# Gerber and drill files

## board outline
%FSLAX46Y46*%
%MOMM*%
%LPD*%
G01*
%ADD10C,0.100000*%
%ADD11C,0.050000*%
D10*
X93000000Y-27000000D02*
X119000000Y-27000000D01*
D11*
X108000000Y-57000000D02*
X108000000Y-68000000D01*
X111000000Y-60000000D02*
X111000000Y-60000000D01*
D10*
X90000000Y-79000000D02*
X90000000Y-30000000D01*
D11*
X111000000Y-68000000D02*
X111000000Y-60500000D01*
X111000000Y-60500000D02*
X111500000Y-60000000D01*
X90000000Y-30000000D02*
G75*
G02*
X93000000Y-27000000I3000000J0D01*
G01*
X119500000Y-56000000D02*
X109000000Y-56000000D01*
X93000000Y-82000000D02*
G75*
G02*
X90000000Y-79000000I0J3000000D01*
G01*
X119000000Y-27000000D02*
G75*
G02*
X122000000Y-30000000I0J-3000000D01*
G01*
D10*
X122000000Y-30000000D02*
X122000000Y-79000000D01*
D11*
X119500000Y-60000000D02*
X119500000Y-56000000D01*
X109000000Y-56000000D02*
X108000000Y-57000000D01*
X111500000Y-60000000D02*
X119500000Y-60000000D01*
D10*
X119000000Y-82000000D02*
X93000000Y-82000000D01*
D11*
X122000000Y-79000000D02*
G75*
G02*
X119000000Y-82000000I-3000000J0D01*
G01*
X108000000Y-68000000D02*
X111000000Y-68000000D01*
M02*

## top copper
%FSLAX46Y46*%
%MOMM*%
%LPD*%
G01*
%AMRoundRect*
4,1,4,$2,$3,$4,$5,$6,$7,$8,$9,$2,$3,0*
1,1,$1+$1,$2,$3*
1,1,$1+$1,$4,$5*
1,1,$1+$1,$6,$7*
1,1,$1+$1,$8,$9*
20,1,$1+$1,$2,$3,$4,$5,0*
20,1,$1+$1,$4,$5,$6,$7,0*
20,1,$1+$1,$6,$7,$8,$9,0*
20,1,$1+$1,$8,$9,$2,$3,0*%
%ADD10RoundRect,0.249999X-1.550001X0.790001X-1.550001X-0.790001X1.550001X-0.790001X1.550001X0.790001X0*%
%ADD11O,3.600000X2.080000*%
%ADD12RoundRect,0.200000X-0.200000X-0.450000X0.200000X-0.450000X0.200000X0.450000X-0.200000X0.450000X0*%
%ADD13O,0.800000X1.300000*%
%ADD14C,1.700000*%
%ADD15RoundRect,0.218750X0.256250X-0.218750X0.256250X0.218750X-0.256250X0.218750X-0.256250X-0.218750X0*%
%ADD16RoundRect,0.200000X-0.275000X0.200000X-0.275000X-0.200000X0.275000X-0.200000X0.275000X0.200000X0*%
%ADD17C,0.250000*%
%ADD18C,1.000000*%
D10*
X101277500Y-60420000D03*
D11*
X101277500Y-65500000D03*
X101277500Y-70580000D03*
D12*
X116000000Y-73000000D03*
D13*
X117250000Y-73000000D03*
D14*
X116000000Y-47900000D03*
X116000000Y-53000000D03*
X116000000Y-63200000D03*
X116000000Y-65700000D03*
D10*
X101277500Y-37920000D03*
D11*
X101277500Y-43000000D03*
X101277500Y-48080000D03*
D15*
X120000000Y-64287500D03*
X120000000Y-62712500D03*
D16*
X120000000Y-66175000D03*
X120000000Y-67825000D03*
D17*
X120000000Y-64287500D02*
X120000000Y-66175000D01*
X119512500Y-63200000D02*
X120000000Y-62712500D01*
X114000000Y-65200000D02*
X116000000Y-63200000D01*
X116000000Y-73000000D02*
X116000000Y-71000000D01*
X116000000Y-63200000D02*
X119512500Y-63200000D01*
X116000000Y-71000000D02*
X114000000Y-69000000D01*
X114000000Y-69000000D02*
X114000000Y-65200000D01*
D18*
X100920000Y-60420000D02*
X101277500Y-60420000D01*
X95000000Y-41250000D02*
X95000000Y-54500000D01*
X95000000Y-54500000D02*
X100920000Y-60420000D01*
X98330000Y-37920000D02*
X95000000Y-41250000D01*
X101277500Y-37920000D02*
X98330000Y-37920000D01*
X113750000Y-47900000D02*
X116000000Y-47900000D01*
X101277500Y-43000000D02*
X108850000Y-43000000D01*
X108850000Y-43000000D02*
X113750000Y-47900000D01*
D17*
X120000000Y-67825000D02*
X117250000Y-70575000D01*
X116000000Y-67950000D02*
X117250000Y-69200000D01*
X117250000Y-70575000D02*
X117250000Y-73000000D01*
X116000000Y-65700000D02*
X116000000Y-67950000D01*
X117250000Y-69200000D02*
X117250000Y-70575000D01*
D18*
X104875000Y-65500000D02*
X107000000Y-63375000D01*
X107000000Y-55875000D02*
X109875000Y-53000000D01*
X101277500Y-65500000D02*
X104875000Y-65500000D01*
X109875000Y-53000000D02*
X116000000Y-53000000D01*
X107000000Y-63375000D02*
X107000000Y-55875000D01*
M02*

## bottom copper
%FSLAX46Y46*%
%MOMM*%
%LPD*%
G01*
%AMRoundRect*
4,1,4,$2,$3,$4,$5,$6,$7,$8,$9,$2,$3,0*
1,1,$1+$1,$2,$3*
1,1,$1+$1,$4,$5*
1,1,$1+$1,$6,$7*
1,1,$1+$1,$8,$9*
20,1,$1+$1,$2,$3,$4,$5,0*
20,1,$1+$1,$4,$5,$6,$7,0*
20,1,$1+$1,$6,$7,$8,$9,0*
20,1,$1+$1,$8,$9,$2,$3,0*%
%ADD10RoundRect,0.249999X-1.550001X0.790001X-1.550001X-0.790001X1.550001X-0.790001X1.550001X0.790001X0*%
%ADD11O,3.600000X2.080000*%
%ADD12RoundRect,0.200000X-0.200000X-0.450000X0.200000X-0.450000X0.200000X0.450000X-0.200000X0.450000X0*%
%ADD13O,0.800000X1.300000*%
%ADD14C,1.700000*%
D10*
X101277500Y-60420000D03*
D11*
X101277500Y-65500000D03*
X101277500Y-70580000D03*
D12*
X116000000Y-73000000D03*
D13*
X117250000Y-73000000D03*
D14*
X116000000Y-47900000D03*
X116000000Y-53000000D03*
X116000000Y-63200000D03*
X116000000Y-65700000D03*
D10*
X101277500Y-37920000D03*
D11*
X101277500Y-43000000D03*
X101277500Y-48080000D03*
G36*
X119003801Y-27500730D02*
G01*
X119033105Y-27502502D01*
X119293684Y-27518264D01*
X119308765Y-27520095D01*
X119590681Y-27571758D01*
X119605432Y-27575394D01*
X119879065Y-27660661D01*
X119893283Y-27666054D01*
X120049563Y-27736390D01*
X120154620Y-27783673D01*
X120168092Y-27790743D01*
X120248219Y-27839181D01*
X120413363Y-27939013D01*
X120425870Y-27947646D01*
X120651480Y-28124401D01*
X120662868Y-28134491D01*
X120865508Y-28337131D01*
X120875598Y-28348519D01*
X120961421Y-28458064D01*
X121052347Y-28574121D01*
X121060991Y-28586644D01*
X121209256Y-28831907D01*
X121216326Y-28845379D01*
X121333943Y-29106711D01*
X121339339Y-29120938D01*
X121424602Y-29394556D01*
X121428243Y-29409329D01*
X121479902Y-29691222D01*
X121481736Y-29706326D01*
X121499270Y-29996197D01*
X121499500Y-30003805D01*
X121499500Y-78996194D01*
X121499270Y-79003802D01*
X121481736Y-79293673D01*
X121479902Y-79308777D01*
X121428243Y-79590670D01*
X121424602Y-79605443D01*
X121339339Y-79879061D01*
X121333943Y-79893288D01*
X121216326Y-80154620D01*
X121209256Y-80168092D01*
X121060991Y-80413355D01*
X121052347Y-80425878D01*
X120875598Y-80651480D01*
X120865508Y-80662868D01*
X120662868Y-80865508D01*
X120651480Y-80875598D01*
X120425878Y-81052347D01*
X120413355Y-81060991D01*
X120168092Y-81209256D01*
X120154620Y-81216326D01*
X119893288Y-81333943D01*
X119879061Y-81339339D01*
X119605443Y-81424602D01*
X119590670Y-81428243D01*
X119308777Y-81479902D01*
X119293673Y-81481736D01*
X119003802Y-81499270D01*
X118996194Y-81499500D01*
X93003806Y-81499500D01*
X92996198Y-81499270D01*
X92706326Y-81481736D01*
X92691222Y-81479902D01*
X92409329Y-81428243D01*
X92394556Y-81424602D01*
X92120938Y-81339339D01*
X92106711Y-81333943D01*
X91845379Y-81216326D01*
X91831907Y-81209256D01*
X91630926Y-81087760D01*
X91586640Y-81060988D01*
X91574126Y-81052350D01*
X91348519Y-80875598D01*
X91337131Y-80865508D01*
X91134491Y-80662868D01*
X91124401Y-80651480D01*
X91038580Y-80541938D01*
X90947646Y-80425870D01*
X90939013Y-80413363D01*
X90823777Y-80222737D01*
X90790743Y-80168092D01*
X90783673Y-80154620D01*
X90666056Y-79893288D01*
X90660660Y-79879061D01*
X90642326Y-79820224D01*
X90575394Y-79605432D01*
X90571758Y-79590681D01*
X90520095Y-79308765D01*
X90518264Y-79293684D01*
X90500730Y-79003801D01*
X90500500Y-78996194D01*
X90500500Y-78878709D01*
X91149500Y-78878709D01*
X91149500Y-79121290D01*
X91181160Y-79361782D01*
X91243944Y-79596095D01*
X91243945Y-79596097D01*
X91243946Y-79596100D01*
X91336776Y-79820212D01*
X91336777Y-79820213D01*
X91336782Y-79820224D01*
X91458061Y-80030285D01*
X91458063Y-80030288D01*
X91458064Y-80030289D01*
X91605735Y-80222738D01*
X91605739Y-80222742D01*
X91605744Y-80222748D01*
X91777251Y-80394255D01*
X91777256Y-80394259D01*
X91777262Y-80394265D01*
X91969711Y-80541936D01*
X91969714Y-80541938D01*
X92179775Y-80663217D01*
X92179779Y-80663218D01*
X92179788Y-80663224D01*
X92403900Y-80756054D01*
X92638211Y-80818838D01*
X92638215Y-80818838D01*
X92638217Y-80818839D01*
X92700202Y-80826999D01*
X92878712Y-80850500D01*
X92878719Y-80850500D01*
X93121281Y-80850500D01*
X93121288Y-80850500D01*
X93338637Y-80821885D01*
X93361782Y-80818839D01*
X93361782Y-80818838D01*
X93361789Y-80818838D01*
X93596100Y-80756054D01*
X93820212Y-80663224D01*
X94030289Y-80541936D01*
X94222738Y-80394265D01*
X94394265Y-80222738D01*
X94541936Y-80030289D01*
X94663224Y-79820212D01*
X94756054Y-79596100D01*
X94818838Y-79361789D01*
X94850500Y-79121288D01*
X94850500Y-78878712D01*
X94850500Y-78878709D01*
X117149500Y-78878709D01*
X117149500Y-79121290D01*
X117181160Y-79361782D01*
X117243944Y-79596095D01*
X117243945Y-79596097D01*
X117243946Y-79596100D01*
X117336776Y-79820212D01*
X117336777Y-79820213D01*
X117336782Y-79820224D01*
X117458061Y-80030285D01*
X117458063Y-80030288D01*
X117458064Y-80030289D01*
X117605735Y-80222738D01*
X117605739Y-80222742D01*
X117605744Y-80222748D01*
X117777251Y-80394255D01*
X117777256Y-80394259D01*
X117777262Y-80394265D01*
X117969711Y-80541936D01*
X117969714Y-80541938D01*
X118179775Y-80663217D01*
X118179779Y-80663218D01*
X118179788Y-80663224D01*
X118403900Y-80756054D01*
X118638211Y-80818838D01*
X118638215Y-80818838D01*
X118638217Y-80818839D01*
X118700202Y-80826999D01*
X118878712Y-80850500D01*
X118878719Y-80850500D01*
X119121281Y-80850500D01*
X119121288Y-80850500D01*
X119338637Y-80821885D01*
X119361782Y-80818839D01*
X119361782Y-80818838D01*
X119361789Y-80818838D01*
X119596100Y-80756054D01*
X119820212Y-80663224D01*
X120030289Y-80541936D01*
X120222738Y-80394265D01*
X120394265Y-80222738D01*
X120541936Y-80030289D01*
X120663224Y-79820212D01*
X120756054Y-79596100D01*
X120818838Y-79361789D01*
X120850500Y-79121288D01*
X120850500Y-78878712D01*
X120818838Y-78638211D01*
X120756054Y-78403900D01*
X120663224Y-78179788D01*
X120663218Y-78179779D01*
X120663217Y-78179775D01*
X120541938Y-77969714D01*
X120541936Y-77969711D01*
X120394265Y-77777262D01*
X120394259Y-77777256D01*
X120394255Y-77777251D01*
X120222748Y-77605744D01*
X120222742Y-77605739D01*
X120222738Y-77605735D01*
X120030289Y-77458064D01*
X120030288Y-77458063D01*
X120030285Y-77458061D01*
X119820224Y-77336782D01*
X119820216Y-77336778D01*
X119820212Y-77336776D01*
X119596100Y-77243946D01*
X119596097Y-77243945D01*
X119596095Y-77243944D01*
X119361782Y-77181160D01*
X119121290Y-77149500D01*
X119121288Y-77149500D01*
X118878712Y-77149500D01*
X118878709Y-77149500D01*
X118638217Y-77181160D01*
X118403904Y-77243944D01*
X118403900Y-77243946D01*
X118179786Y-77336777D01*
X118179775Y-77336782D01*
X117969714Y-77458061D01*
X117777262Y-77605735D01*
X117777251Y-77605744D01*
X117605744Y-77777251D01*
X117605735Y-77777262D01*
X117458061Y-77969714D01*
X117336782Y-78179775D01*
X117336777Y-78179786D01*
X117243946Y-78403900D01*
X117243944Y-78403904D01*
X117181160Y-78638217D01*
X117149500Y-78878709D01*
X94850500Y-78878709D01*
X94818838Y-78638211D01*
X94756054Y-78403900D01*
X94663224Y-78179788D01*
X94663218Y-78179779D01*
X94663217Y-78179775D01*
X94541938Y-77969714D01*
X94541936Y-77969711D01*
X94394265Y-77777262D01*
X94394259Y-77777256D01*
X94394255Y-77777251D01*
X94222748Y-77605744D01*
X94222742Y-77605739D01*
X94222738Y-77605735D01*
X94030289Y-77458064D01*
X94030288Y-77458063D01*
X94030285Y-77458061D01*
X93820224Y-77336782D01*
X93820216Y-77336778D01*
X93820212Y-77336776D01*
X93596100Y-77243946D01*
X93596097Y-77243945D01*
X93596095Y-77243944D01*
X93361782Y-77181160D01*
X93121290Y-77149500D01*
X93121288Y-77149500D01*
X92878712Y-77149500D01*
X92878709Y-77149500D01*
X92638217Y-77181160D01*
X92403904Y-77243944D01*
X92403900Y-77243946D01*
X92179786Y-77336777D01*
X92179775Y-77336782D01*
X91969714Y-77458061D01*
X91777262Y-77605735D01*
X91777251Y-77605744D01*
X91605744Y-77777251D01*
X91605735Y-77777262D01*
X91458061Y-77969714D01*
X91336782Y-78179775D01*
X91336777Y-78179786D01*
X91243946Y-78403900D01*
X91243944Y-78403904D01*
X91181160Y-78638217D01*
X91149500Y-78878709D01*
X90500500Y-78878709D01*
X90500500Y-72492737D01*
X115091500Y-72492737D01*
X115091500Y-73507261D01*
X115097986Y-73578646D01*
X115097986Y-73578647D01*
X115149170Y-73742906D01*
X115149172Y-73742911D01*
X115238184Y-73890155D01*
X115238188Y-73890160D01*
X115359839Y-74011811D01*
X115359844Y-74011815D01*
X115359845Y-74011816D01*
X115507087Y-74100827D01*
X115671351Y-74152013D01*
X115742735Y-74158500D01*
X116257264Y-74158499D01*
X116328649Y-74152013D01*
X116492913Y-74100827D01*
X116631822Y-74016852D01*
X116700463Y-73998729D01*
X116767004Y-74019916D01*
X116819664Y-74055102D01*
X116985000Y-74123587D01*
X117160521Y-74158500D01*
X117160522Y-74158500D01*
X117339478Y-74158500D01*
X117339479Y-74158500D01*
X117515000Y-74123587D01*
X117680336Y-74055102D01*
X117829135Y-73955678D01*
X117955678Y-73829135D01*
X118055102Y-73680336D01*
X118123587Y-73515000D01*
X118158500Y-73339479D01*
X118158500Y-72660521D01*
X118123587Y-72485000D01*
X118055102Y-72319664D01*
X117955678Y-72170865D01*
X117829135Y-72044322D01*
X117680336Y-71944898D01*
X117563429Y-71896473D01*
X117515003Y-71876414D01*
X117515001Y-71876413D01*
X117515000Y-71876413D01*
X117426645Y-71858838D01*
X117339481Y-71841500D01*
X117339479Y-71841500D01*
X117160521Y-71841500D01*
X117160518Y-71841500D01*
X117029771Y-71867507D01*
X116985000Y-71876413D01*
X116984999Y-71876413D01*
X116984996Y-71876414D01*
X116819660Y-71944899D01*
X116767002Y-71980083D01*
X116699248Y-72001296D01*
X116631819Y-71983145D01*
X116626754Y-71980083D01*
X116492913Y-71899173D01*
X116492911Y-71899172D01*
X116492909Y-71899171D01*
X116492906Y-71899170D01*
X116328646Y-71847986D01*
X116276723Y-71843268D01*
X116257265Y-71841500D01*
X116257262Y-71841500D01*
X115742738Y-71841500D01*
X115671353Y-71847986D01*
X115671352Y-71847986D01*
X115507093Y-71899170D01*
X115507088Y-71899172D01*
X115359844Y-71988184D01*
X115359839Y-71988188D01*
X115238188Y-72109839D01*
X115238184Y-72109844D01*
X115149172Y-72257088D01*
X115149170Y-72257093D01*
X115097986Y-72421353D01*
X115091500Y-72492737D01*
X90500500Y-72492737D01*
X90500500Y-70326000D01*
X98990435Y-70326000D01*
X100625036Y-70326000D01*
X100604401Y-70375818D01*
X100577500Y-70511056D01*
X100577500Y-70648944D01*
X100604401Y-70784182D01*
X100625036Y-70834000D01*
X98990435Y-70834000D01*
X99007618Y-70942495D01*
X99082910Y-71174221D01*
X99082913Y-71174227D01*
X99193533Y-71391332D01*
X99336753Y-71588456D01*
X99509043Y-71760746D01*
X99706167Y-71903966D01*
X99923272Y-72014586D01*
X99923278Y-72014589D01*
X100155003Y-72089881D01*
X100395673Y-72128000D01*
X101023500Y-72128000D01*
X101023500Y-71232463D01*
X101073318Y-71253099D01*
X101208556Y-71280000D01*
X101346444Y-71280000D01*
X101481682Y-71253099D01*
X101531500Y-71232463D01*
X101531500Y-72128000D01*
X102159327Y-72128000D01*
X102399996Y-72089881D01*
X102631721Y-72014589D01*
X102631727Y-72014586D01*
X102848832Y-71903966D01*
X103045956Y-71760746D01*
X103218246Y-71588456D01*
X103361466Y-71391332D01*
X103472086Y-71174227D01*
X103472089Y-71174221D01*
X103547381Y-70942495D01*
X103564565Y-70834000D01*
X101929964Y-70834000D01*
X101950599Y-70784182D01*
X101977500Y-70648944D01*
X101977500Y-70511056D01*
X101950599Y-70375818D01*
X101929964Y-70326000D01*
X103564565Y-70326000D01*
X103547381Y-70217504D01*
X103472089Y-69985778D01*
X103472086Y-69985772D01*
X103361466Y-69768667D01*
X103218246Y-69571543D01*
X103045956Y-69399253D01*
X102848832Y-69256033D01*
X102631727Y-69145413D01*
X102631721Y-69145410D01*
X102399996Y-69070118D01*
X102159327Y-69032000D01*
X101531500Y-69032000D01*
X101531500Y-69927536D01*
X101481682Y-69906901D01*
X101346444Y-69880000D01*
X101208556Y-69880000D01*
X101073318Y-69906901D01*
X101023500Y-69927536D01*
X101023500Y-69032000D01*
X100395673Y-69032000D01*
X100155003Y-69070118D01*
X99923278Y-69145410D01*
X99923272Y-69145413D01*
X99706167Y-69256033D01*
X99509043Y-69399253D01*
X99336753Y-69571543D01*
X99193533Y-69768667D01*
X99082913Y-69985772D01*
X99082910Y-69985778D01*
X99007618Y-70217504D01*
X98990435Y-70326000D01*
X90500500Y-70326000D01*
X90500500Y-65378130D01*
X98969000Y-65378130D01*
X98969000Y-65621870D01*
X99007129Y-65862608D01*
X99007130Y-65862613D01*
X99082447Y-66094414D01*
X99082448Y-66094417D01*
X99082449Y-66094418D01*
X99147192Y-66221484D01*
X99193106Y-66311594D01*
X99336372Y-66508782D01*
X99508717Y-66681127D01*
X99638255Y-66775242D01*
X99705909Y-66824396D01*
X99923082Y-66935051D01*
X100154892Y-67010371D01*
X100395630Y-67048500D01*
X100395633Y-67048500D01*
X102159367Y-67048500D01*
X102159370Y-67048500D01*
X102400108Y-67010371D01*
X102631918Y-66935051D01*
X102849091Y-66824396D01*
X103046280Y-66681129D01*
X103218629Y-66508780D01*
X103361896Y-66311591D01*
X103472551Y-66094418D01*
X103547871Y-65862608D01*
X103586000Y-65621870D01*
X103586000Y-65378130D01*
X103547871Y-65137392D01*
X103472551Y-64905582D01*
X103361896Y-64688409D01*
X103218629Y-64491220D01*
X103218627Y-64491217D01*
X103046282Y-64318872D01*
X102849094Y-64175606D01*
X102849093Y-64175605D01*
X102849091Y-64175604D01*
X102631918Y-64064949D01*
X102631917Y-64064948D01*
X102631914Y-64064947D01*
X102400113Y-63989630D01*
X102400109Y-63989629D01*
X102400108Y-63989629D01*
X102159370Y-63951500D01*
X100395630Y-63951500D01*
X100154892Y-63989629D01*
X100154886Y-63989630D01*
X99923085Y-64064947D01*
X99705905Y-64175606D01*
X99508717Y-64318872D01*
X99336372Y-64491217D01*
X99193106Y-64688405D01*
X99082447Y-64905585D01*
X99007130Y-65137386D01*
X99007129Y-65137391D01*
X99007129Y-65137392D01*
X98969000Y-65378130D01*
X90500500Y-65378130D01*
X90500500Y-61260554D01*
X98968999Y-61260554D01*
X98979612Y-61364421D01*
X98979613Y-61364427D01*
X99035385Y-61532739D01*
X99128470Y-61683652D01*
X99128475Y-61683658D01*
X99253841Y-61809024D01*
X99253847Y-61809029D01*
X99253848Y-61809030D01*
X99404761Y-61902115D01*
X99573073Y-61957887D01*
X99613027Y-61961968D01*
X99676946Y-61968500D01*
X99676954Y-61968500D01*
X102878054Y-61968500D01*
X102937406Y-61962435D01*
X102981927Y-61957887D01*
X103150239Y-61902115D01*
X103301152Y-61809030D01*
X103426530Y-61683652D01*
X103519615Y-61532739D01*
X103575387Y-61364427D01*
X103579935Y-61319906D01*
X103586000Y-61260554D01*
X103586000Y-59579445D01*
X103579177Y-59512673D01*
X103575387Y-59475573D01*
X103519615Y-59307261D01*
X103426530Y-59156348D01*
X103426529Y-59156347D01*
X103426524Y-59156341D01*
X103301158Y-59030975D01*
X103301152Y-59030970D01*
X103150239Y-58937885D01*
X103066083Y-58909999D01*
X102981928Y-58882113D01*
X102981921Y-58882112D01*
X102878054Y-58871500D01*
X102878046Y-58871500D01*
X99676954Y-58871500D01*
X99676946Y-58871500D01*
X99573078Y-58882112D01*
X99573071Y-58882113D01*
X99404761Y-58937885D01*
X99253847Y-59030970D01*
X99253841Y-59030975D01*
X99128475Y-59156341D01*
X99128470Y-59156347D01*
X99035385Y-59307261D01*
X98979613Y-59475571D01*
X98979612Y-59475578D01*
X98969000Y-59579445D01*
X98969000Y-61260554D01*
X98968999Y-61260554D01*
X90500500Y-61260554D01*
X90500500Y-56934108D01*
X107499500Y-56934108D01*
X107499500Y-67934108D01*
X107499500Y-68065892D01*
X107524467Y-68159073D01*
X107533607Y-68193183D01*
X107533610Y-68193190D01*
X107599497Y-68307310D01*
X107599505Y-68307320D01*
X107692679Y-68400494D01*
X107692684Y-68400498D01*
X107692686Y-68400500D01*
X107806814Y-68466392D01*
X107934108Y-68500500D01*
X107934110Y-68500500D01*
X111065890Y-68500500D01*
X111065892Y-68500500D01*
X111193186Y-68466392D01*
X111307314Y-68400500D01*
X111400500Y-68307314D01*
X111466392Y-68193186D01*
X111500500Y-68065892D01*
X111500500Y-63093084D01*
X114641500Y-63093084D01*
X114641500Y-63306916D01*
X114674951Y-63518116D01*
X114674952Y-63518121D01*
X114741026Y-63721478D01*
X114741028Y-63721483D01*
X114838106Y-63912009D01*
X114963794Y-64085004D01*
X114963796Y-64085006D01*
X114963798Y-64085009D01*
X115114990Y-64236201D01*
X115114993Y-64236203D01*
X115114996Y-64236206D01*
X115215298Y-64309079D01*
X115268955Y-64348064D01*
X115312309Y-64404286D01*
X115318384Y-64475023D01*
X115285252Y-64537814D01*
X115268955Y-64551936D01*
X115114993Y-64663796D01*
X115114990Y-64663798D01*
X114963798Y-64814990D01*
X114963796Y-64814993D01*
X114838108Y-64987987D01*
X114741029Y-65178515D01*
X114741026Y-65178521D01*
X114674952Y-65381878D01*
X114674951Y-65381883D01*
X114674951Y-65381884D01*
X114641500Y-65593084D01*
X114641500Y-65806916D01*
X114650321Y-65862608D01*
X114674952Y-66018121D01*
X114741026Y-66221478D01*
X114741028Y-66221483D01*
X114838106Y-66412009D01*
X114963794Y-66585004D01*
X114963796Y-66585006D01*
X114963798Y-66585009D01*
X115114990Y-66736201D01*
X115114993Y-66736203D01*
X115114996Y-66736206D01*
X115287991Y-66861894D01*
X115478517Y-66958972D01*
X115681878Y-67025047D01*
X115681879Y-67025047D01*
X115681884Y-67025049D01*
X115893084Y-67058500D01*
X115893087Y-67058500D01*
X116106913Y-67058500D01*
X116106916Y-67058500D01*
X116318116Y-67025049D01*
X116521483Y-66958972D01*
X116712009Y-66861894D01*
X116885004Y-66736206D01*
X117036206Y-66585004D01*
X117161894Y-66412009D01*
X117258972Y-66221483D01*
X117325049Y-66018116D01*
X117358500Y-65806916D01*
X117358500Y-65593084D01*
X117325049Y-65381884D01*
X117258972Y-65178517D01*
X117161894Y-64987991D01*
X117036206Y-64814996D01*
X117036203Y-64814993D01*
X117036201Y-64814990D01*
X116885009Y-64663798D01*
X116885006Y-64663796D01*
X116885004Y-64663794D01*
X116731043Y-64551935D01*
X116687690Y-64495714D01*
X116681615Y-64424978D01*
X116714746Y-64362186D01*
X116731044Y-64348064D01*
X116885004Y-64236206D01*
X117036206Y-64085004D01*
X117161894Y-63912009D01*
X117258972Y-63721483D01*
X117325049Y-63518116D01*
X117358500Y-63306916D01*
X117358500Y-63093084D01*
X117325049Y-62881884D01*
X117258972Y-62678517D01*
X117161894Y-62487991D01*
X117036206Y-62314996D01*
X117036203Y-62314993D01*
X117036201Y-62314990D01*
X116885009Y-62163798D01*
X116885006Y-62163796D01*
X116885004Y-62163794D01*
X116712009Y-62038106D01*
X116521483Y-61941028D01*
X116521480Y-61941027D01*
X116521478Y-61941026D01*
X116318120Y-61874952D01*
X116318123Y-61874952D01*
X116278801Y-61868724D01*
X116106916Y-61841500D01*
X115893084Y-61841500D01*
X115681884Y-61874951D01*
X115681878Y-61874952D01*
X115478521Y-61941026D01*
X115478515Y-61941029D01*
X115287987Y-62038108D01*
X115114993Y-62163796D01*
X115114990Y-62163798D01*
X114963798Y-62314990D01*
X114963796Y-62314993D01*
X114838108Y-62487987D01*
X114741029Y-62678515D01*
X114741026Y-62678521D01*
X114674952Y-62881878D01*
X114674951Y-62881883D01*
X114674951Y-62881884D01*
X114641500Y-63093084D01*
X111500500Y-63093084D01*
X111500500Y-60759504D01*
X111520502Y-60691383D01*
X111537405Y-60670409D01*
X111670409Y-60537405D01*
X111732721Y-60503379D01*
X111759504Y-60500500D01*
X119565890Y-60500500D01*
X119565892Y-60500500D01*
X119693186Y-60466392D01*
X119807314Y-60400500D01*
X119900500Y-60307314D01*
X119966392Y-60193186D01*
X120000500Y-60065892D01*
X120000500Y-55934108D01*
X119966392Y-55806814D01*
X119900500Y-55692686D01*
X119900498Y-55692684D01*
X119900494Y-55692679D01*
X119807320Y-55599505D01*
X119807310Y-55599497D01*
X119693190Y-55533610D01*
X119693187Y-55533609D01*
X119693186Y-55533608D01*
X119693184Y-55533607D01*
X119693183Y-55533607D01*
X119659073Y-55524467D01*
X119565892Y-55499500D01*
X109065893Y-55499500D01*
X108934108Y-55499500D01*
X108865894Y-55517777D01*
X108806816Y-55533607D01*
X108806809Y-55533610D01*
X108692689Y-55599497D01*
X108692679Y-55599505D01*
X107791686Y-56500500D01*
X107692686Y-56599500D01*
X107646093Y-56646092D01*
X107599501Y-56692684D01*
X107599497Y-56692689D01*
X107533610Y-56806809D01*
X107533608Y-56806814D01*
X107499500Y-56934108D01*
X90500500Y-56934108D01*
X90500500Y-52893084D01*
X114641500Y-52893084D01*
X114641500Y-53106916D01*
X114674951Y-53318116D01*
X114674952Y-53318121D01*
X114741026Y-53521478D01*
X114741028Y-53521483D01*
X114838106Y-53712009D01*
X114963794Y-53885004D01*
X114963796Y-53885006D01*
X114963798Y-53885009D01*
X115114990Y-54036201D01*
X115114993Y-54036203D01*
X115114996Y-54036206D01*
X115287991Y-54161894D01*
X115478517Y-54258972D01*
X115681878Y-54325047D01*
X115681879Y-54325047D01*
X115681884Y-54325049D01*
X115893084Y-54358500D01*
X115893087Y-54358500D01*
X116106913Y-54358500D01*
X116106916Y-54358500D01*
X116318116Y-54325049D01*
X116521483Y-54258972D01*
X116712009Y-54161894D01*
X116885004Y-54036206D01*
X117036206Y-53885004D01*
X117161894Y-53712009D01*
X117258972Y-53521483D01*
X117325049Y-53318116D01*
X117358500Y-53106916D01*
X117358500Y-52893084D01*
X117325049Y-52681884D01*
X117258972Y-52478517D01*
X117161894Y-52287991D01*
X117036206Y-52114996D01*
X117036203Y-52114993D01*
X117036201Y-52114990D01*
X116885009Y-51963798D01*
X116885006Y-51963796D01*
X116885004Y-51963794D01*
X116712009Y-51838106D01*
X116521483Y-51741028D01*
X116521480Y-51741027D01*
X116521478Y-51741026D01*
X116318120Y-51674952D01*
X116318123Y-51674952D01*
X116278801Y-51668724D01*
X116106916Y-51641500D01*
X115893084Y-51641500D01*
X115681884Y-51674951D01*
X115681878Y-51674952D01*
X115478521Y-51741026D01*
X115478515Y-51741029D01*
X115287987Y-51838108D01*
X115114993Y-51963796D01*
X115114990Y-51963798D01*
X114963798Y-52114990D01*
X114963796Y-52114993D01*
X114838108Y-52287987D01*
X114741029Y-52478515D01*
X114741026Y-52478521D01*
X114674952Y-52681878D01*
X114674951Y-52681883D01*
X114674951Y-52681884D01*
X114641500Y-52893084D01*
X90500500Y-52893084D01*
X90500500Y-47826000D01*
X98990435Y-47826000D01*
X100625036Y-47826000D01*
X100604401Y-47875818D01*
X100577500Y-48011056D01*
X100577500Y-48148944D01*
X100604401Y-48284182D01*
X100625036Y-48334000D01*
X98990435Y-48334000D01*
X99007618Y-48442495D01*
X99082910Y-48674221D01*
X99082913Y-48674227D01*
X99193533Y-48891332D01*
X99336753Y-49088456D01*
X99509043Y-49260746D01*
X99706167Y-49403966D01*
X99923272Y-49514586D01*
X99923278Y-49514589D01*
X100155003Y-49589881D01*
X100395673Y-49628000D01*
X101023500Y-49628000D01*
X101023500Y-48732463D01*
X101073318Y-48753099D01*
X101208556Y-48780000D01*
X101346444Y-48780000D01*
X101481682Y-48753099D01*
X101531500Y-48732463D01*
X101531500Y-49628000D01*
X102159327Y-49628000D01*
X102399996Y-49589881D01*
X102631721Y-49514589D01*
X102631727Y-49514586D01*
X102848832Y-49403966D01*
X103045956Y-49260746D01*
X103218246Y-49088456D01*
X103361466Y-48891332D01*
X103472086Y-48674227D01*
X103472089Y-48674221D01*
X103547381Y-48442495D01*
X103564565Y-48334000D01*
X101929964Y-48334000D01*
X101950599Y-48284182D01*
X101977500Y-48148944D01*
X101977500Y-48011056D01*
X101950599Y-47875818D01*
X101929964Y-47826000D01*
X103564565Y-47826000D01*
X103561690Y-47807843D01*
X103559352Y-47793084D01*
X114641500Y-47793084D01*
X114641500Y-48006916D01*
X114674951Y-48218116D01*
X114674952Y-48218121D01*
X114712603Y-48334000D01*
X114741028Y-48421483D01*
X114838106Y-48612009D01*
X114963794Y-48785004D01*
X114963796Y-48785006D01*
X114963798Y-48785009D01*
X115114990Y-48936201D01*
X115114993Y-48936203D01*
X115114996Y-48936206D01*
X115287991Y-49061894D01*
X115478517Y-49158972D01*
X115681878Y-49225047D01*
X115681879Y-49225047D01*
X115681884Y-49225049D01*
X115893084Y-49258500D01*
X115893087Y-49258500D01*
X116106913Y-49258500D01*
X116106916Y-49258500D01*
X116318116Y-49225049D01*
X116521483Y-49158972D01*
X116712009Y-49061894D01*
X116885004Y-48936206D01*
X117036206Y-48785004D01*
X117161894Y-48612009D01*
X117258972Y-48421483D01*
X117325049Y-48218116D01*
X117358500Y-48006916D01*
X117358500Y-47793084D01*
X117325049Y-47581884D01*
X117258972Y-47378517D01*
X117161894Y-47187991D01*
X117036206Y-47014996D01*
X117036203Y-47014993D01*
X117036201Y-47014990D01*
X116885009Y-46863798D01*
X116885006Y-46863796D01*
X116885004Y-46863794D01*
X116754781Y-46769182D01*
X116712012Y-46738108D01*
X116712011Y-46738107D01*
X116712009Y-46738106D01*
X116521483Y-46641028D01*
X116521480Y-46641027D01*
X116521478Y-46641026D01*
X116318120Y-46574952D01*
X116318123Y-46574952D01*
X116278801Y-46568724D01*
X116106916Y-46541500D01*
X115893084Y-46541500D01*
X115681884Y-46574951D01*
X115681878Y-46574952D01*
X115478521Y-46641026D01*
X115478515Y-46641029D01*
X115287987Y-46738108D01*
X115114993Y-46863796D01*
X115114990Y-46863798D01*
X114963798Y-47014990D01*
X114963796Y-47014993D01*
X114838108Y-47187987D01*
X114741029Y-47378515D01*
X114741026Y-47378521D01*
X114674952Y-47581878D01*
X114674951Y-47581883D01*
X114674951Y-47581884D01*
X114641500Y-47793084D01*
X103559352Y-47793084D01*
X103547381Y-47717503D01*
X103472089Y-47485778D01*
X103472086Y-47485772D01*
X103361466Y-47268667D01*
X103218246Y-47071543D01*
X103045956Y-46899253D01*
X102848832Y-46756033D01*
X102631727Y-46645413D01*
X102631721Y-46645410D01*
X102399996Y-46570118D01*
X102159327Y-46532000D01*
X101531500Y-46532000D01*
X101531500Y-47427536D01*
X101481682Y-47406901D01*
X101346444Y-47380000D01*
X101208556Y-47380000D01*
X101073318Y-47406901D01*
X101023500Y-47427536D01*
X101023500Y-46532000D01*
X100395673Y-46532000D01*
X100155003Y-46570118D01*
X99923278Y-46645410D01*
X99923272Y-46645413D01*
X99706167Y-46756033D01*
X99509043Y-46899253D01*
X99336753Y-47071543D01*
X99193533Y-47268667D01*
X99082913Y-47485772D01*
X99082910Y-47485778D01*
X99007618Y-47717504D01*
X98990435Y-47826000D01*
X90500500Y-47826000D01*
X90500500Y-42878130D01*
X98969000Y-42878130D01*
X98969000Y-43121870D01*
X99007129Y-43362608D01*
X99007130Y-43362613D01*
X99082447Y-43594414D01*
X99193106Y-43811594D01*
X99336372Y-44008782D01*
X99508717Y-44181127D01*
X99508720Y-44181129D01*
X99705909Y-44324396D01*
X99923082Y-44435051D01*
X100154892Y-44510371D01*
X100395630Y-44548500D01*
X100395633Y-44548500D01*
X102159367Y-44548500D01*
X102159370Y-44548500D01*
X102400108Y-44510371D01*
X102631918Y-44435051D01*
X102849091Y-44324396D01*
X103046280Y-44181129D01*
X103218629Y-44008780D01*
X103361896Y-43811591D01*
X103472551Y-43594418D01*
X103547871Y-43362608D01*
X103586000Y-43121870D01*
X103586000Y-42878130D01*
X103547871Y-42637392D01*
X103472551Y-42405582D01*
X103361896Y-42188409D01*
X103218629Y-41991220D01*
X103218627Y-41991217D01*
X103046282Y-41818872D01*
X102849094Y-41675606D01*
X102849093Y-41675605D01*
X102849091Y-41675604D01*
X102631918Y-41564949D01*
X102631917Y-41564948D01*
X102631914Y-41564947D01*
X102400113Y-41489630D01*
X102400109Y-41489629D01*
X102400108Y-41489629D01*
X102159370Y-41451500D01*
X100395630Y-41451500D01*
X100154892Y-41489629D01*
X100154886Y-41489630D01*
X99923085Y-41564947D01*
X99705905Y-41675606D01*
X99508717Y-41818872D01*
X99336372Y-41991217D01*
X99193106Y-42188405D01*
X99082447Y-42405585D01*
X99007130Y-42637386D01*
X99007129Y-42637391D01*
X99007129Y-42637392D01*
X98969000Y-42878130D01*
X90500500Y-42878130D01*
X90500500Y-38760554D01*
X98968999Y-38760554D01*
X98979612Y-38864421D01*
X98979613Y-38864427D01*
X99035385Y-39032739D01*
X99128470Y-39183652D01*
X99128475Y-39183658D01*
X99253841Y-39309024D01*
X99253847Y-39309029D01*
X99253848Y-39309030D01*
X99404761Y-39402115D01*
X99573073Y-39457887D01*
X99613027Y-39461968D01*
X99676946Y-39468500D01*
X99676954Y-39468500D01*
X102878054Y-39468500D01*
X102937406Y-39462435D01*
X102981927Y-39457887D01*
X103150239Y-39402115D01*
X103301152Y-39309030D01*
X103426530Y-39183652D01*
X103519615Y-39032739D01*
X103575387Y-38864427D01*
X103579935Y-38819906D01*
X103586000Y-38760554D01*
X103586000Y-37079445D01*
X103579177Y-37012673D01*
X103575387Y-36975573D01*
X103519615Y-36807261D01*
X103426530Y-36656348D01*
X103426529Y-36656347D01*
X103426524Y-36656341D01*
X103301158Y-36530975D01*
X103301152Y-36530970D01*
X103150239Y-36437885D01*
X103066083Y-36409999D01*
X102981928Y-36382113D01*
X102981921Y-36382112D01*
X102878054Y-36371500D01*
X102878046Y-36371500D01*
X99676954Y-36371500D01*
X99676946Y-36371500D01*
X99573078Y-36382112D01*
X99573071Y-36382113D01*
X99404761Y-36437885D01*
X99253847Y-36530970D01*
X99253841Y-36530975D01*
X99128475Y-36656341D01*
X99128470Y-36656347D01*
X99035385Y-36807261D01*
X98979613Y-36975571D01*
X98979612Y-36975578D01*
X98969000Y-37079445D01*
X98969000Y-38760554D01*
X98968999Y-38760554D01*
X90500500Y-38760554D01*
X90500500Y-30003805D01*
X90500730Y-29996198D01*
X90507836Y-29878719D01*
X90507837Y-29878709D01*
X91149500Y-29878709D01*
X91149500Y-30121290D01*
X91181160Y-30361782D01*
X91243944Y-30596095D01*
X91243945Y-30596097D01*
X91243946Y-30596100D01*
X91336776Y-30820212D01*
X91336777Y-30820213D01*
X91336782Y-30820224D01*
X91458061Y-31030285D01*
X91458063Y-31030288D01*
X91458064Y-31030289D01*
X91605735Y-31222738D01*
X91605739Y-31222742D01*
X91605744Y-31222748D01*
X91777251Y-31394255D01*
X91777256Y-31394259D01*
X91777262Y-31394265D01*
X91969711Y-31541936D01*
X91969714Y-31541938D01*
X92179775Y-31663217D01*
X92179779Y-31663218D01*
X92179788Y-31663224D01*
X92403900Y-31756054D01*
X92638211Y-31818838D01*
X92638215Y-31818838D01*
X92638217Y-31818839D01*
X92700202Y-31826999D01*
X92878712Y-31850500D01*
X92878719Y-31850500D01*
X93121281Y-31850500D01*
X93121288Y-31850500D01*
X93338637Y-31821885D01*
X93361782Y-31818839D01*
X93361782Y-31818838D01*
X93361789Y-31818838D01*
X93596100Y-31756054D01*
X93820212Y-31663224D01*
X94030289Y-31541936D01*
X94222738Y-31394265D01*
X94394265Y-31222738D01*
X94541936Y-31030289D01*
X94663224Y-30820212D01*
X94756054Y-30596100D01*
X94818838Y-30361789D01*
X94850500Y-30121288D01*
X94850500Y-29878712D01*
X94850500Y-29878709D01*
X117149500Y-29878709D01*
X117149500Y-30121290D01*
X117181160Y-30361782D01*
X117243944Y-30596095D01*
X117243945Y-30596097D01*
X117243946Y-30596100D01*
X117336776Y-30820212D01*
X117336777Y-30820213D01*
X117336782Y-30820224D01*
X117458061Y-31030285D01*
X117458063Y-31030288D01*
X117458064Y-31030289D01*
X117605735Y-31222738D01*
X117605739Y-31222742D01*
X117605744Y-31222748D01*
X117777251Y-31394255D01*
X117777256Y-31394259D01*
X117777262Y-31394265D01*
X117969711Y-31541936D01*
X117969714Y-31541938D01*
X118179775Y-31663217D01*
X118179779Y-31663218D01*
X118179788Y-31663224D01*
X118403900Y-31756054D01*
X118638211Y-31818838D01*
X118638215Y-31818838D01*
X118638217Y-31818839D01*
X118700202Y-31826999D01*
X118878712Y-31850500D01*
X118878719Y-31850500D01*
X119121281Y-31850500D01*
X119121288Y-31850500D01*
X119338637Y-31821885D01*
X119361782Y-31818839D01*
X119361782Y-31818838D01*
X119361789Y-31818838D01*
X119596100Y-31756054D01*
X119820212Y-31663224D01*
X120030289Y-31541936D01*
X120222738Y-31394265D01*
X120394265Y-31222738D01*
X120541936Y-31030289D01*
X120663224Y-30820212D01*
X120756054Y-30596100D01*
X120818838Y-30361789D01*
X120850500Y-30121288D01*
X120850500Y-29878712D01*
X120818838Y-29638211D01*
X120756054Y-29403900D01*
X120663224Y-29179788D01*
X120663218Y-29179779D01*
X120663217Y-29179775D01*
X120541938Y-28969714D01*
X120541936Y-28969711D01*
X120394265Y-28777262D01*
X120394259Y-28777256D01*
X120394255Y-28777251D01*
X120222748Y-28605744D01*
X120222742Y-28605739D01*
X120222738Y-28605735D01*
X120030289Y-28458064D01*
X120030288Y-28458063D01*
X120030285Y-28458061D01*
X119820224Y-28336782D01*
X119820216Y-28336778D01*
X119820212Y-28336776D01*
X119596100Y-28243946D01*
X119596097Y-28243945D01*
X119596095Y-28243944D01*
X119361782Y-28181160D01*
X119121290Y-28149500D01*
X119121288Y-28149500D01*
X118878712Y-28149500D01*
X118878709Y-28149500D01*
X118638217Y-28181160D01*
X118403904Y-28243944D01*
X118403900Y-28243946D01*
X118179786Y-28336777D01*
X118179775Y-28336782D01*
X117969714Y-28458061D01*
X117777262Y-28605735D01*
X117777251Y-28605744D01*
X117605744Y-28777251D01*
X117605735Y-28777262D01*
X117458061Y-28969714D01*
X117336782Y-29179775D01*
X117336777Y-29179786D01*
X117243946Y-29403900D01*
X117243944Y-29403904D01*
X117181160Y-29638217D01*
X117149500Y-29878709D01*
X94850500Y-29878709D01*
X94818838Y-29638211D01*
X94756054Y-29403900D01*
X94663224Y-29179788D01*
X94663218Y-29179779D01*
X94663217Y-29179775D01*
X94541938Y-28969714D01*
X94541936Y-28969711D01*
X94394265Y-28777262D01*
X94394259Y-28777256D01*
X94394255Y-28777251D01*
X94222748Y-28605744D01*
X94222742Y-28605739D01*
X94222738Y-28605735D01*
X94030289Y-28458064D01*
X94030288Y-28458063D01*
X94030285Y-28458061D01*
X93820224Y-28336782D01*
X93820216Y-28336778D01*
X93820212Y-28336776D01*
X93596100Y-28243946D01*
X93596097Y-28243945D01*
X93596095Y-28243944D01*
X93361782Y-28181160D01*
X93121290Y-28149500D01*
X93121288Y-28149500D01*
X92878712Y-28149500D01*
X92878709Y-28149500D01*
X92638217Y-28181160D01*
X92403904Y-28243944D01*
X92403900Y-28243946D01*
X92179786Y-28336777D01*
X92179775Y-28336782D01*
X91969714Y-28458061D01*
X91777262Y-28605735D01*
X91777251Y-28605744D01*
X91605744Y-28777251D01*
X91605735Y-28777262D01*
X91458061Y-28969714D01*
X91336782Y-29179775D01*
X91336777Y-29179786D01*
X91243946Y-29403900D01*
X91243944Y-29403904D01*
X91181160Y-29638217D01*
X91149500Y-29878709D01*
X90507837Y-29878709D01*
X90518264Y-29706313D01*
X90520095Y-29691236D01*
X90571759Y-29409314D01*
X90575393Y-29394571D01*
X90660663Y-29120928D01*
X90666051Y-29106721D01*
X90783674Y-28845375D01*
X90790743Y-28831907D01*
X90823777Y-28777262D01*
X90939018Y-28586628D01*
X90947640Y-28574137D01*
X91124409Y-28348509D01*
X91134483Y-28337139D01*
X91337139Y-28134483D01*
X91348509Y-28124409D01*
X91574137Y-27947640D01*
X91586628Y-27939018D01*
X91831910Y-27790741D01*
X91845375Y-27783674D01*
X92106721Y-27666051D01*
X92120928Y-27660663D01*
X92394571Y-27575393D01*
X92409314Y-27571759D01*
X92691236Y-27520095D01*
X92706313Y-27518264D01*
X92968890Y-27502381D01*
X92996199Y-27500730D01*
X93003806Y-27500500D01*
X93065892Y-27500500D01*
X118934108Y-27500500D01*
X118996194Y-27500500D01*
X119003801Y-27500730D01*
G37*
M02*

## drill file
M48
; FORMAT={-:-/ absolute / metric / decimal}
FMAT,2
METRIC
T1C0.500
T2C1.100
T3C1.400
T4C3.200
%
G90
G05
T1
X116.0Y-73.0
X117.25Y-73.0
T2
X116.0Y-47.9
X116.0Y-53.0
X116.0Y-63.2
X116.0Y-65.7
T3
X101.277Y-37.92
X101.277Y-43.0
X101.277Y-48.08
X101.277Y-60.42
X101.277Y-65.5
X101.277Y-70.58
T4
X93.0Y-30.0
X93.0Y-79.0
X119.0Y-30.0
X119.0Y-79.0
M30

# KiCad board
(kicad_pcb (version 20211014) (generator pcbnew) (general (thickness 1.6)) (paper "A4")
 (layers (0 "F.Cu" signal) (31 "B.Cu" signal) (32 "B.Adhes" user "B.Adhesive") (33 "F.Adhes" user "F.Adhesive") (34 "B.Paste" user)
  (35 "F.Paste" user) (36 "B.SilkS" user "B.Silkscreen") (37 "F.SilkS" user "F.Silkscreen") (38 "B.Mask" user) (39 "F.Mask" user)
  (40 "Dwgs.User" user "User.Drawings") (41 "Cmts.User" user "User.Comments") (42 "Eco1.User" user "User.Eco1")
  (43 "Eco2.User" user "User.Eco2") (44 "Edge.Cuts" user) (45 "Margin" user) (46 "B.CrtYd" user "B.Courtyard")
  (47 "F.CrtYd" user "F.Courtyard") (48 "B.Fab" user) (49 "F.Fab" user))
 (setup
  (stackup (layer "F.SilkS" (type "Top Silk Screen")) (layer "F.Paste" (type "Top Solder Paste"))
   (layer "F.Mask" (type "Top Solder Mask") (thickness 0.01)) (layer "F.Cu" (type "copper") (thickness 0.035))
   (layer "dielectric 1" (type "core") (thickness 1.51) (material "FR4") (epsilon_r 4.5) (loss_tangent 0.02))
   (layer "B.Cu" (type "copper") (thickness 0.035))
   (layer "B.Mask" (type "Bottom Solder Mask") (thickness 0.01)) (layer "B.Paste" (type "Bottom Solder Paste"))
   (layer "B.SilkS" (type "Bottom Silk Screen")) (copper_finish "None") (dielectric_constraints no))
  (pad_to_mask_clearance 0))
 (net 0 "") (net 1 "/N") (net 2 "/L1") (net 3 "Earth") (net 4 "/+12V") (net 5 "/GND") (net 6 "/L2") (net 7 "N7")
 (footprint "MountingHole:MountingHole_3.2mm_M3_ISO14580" (layer "F.Cu") (at 119 79)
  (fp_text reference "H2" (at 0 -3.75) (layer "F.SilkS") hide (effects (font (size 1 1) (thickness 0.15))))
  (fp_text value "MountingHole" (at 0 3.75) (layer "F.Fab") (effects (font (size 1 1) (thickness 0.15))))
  (pad "" np_thru_hole circle (at 0 0) (size 3.2 3.2) (drill 3.2) (layers *.Cu *.Mask)))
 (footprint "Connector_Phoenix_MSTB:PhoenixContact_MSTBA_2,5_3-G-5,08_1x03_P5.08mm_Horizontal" (layer "F.Cu") (at 101.2775 60.42 -90)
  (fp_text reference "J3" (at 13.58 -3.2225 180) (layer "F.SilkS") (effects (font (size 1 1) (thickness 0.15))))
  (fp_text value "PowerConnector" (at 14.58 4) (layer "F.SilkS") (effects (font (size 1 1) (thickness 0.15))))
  (pad "1" thru_hole roundrect (at 0 0 270) (size 2.08 3.6) (drill 1.4) (layers *.Cu *.Mask) (roundrect_rratio 0.120192) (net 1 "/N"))
  (pad "2" thru_hole oval (at 5.08 0 270) (size 2.08 3.6) (drill 1.4) (layers *.Cu *.Mask) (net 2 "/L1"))
  (pad "3" thru_hole oval (at 10.16 0 270) (size 2.08 3.6) (drill 1.4) (layers *.Cu *.Mask) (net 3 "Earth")))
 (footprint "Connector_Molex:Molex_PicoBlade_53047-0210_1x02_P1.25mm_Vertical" (layer "F.Cu") (at 116 73)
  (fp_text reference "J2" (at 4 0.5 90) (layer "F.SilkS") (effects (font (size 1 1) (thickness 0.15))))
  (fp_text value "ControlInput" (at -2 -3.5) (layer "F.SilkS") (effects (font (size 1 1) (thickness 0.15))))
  (pad "1" thru_hole roundrect (at 0 0) (size 0.8 1.3) (drill 0.5) (layers *.Cu *.Mask) (roundrect_rratio 0.25) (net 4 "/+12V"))
  (pad "2" thru_hole oval (at 1.25 0) (size 0.8 1.3) (drill 0.5) (layers *.Cu *.Mask) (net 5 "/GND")))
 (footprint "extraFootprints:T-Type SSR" (layer "F.Cu") (at 116 53 -90)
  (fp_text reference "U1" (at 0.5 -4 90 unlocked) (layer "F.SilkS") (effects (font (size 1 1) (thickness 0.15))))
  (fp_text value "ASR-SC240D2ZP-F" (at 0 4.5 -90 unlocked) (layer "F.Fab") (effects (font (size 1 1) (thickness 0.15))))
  (pad "1" thru_hole circle (at -5.1 0 270) (size 1.7 1.7) (drill 1.1) (layers *.Cu *.Mask) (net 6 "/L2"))
  (pad "2" thru_hole circle (at 0 0 270) (size 1.7 1.7) (drill 1.1) (layers *.Cu *.Mask) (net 2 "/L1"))
  (pad "3" thru_hole circle (at 10.2 0 270) (size 1.7 1.7) (drill 1.1) (layers *.Cu *.Mask) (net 4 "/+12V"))
  (pad "4" thru_hole circle (at 12.7 0 270) (size 1.7 1.7) (drill 1.1) (layers *.Cu *.Mask) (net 5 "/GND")))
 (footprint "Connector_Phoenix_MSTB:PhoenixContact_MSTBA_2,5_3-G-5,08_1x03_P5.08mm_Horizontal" (layer "F.Cu") (at 101.2775 37.92 -90)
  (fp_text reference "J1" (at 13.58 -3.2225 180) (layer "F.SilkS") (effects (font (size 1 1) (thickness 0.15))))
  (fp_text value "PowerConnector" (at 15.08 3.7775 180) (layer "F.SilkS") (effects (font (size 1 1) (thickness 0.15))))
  (pad "1" thru_hole roundrect (at 0 0 270) (size 2.08 3.6) (drill 1.4) (layers *.Cu *.Mask) (roundrect_rratio 0.120192) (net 1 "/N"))
  (pad "2" thru_hole oval (at 5.08 0 270) (size 2.08 3.6) (drill 1.4) (layers *.Cu *.Mask) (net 6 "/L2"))
  (pad "3" thru_hole oval (at 10.16 0 270) (size 2.08 3.6) (drill 1.4) (layers *.Cu *.Mask) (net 3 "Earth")))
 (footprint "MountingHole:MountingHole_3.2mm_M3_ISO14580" (layer "F.Cu") (at 93 79)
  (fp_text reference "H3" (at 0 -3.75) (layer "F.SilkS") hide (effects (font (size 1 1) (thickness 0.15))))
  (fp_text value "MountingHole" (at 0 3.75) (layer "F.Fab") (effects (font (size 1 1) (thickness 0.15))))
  (pad "" np_thru_hole circle (at 0 0) (size 3.2 3.2) (drill 3.2) (layers *.Cu *.Mask)))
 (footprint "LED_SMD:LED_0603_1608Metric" (layer "F.Cu") (at 120 63.5 90)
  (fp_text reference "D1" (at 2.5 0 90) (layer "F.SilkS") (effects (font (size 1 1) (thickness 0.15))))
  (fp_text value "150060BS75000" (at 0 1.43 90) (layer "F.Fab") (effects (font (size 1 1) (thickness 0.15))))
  (pad "1" smd roundrect (at -0.7875 0 90) (size 0.875 0.95) (layers "F.Cu" "F.Paste" "F.Mask") (roundrect_rratio 0.25) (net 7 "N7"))
  (pad "2" smd roundrect (at 0.7875 0 90) (size 0.875 0.95) (layers "F.Cu" "F.Paste" "F.Mask") (roundrect_rratio 0.25) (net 4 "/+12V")))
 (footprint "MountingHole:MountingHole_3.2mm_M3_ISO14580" (layer "F.Cu") (at 93 30)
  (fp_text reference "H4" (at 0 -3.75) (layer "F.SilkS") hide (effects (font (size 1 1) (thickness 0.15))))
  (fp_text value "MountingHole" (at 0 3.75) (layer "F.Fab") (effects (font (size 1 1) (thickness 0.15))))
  (pad "" np_thru_hole circle (at 0 0) (size 3.2 3.2) (drill 3.2) (layers *.Cu *.Mask)))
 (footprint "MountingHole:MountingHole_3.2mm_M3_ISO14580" (layer "F.Cu") (at 119 30)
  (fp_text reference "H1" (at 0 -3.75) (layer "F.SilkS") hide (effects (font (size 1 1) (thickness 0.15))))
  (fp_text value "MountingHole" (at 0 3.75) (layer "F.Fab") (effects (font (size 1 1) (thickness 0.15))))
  (pad "" np_thru_hole circle (at 0 0) (size 3.2 3.2) (drill 3.2) (layers *.Cu *.Mask)))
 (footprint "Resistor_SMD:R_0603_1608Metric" (layer "F.Cu") (at 120 67 -90)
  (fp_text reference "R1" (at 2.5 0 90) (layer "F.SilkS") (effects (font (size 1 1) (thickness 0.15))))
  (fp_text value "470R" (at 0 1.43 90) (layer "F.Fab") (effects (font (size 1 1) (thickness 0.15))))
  (pad "1" smd roundrect (at -0.825 0 270) (size 0.8 0.95) (layers "F.Cu" "F.Paste" "F.Mask") (roundrect_rratio 0.25) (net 7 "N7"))
  (pad "2" smd roundrect (at 0.825 0 270) (size 0.8 0.95) (layers "F.Cu" "F.Paste" "F.Mask") (roundrect_rratio 0.25) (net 5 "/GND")))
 (gr_line (start 93 27) (end 119 27) (layer "Edge.Cuts") (width 0.1))
 (gr_line (start 108 57) (end 108 68) (layer "Edge.Cuts") (width 0.05))
 (gr_line (start 111 60) (end 111 60) (layer "Edge.Cuts") (width 0.05))
 (gr_line (start 90 79) (end 90 30) (layer "Edge.Cuts") (width 0.1))
 (gr_line (start 111 68) (end 111 60.5) (layer "Edge.Cuts") (width 0.05))
 (gr_line (start 111 60.5) (end 111.5 60) (layer "Edge.Cuts") (width 0.05))
 (gr_arc (start 90 30) (mid 90.87868 27.87868) (end 93 27) (layer "Edge.Cuts") (width 0.05))
 (gr_line (start 119.5 56) (end 109 56) (layer "Edge.Cuts") (width 0.05))
 (gr_arc (start 93 82) (mid 90.87868 81.12132) (end 90 79) (layer "Edge.Cuts") (width 0.05))
 (gr_arc (start 119 27) (mid 121.12132 27.87868) (end 122 30) (layer "Edge.Cuts") (width 0.05))
 (gr_line (start 122 30) (end 122 79) (layer "Edge.Cuts") (width 0.1))
 (gr_line (start 119.5 60) (end 119.5 56) (layer "Edge.Cuts") (width 0.05))
 (gr_line (start 109 56) (end 108 57) (layer "Edge.Cuts") (width 0.05))
 (gr_line (start 111.5 60) (end 119.5 60) (layer "Edge.Cuts") (width 0.05))
 (gr_line (start 119 82) (end 93 82) (layer "Edge.Cuts") (width 0.1))
 (gr_arc (start 122 79) (mid 121.12132 81.12132) (end 119 82) (layer "Edge.Cuts") (width 0.05))
 (gr_line (start 108 68) (end 111 68) (layer "Edge.Cuts") (width 0.05))
 (segment (start 120 64.2875) (end 120 66.175) (width 0.25) (layer "F.Cu") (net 7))
 (segment (start 119.5125 63.2) (end 120 62.7125) (width 0.25) (layer "F.Cu") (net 4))
 (segment (start 114 65.2) (end 116 63.2) (width 0.25) (layer "F.Cu") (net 4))
 (segment (start 116 73) (end 116 71) (width 0.25) (layer "F.Cu") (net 4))
 (segment (start 116 63.2) (end 119.5125 63.2) (width 0.25) (layer "F.Cu") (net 4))
 (segment (start 116 71) (end 114 69) (width 0.25) (layer "F.Cu") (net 4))
 (segment (start 114 69) (end 114 65.2) (width 0.25) (layer "F.Cu") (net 4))
 (segment (start 100.92 60.42) (end 101.2775 60.42) (width 1) (layer "F.Cu") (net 1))
 (segment (start 95 41.25) (end 95 54.5) (width 1) (layer "F.Cu") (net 1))
 (segment (start 95 54.5) (end 100.92 60.42) (width 1) (layer "F.Cu") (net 1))
 (segment (start 98.33 37.92) (end 95 41.25) (width 1) (layer "F.Cu") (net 1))
 (segment (start 101.2775 37.92) (end 98.33 37.92) (width 1) (layer "F.Cu") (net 1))
 (segment (start 113.75 47.9) (end 116 47.9) (width 1) (layer "F.Cu") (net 6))
 (segment (start 101.2775 43) (end 108.85 43) (width 1) (layer "F.Cu") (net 6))
 (segment (start 108.85 43) (end 113.75 47.9) (width 1) (layer "F.Cu") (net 6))
 (segment (start 120 67.825) (end 117.25 70.575) (width 0.25) (layer "F.Cu") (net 5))
 (segment (start 116 67.95) (end 117.25 69.2) (width 0.25) (layer "F.Cu") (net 5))
 (segment (start 117.25 70.575) (end 117.25 73) (width 0.25) (layer "F.Cu") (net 5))
 (segment (start 116 65.7) (end 116 67.95) (width 0.25) (layer "F.Cu") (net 5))
 (segment (start 117.25 69.2) (end 117.25 70.575) (width 0.25) (layer "F.Cu") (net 5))
 (segment (start 104.875 65.5) (end 107 63.375) (width 1) (layer "F.Cu") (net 2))
 (segment (start 107 55.875) (end 109.875 53) (width 1) (layer "F.Cu") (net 2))
 (segment (start 101.2775 65.5) (end 104.875 65.5) (width 1) (layer "F.Cu") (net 2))
 (segment (start 109.875 53) (end 116 53) (width 1) (layer "F.Cu") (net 2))
 (segment (start 107 63.375) (end 107 55.875) (width 1) (layer "F.Cu") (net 2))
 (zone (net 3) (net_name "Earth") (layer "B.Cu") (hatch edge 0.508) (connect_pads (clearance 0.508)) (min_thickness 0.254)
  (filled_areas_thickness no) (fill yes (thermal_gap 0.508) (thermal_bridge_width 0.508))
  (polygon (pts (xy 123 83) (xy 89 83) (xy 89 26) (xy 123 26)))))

